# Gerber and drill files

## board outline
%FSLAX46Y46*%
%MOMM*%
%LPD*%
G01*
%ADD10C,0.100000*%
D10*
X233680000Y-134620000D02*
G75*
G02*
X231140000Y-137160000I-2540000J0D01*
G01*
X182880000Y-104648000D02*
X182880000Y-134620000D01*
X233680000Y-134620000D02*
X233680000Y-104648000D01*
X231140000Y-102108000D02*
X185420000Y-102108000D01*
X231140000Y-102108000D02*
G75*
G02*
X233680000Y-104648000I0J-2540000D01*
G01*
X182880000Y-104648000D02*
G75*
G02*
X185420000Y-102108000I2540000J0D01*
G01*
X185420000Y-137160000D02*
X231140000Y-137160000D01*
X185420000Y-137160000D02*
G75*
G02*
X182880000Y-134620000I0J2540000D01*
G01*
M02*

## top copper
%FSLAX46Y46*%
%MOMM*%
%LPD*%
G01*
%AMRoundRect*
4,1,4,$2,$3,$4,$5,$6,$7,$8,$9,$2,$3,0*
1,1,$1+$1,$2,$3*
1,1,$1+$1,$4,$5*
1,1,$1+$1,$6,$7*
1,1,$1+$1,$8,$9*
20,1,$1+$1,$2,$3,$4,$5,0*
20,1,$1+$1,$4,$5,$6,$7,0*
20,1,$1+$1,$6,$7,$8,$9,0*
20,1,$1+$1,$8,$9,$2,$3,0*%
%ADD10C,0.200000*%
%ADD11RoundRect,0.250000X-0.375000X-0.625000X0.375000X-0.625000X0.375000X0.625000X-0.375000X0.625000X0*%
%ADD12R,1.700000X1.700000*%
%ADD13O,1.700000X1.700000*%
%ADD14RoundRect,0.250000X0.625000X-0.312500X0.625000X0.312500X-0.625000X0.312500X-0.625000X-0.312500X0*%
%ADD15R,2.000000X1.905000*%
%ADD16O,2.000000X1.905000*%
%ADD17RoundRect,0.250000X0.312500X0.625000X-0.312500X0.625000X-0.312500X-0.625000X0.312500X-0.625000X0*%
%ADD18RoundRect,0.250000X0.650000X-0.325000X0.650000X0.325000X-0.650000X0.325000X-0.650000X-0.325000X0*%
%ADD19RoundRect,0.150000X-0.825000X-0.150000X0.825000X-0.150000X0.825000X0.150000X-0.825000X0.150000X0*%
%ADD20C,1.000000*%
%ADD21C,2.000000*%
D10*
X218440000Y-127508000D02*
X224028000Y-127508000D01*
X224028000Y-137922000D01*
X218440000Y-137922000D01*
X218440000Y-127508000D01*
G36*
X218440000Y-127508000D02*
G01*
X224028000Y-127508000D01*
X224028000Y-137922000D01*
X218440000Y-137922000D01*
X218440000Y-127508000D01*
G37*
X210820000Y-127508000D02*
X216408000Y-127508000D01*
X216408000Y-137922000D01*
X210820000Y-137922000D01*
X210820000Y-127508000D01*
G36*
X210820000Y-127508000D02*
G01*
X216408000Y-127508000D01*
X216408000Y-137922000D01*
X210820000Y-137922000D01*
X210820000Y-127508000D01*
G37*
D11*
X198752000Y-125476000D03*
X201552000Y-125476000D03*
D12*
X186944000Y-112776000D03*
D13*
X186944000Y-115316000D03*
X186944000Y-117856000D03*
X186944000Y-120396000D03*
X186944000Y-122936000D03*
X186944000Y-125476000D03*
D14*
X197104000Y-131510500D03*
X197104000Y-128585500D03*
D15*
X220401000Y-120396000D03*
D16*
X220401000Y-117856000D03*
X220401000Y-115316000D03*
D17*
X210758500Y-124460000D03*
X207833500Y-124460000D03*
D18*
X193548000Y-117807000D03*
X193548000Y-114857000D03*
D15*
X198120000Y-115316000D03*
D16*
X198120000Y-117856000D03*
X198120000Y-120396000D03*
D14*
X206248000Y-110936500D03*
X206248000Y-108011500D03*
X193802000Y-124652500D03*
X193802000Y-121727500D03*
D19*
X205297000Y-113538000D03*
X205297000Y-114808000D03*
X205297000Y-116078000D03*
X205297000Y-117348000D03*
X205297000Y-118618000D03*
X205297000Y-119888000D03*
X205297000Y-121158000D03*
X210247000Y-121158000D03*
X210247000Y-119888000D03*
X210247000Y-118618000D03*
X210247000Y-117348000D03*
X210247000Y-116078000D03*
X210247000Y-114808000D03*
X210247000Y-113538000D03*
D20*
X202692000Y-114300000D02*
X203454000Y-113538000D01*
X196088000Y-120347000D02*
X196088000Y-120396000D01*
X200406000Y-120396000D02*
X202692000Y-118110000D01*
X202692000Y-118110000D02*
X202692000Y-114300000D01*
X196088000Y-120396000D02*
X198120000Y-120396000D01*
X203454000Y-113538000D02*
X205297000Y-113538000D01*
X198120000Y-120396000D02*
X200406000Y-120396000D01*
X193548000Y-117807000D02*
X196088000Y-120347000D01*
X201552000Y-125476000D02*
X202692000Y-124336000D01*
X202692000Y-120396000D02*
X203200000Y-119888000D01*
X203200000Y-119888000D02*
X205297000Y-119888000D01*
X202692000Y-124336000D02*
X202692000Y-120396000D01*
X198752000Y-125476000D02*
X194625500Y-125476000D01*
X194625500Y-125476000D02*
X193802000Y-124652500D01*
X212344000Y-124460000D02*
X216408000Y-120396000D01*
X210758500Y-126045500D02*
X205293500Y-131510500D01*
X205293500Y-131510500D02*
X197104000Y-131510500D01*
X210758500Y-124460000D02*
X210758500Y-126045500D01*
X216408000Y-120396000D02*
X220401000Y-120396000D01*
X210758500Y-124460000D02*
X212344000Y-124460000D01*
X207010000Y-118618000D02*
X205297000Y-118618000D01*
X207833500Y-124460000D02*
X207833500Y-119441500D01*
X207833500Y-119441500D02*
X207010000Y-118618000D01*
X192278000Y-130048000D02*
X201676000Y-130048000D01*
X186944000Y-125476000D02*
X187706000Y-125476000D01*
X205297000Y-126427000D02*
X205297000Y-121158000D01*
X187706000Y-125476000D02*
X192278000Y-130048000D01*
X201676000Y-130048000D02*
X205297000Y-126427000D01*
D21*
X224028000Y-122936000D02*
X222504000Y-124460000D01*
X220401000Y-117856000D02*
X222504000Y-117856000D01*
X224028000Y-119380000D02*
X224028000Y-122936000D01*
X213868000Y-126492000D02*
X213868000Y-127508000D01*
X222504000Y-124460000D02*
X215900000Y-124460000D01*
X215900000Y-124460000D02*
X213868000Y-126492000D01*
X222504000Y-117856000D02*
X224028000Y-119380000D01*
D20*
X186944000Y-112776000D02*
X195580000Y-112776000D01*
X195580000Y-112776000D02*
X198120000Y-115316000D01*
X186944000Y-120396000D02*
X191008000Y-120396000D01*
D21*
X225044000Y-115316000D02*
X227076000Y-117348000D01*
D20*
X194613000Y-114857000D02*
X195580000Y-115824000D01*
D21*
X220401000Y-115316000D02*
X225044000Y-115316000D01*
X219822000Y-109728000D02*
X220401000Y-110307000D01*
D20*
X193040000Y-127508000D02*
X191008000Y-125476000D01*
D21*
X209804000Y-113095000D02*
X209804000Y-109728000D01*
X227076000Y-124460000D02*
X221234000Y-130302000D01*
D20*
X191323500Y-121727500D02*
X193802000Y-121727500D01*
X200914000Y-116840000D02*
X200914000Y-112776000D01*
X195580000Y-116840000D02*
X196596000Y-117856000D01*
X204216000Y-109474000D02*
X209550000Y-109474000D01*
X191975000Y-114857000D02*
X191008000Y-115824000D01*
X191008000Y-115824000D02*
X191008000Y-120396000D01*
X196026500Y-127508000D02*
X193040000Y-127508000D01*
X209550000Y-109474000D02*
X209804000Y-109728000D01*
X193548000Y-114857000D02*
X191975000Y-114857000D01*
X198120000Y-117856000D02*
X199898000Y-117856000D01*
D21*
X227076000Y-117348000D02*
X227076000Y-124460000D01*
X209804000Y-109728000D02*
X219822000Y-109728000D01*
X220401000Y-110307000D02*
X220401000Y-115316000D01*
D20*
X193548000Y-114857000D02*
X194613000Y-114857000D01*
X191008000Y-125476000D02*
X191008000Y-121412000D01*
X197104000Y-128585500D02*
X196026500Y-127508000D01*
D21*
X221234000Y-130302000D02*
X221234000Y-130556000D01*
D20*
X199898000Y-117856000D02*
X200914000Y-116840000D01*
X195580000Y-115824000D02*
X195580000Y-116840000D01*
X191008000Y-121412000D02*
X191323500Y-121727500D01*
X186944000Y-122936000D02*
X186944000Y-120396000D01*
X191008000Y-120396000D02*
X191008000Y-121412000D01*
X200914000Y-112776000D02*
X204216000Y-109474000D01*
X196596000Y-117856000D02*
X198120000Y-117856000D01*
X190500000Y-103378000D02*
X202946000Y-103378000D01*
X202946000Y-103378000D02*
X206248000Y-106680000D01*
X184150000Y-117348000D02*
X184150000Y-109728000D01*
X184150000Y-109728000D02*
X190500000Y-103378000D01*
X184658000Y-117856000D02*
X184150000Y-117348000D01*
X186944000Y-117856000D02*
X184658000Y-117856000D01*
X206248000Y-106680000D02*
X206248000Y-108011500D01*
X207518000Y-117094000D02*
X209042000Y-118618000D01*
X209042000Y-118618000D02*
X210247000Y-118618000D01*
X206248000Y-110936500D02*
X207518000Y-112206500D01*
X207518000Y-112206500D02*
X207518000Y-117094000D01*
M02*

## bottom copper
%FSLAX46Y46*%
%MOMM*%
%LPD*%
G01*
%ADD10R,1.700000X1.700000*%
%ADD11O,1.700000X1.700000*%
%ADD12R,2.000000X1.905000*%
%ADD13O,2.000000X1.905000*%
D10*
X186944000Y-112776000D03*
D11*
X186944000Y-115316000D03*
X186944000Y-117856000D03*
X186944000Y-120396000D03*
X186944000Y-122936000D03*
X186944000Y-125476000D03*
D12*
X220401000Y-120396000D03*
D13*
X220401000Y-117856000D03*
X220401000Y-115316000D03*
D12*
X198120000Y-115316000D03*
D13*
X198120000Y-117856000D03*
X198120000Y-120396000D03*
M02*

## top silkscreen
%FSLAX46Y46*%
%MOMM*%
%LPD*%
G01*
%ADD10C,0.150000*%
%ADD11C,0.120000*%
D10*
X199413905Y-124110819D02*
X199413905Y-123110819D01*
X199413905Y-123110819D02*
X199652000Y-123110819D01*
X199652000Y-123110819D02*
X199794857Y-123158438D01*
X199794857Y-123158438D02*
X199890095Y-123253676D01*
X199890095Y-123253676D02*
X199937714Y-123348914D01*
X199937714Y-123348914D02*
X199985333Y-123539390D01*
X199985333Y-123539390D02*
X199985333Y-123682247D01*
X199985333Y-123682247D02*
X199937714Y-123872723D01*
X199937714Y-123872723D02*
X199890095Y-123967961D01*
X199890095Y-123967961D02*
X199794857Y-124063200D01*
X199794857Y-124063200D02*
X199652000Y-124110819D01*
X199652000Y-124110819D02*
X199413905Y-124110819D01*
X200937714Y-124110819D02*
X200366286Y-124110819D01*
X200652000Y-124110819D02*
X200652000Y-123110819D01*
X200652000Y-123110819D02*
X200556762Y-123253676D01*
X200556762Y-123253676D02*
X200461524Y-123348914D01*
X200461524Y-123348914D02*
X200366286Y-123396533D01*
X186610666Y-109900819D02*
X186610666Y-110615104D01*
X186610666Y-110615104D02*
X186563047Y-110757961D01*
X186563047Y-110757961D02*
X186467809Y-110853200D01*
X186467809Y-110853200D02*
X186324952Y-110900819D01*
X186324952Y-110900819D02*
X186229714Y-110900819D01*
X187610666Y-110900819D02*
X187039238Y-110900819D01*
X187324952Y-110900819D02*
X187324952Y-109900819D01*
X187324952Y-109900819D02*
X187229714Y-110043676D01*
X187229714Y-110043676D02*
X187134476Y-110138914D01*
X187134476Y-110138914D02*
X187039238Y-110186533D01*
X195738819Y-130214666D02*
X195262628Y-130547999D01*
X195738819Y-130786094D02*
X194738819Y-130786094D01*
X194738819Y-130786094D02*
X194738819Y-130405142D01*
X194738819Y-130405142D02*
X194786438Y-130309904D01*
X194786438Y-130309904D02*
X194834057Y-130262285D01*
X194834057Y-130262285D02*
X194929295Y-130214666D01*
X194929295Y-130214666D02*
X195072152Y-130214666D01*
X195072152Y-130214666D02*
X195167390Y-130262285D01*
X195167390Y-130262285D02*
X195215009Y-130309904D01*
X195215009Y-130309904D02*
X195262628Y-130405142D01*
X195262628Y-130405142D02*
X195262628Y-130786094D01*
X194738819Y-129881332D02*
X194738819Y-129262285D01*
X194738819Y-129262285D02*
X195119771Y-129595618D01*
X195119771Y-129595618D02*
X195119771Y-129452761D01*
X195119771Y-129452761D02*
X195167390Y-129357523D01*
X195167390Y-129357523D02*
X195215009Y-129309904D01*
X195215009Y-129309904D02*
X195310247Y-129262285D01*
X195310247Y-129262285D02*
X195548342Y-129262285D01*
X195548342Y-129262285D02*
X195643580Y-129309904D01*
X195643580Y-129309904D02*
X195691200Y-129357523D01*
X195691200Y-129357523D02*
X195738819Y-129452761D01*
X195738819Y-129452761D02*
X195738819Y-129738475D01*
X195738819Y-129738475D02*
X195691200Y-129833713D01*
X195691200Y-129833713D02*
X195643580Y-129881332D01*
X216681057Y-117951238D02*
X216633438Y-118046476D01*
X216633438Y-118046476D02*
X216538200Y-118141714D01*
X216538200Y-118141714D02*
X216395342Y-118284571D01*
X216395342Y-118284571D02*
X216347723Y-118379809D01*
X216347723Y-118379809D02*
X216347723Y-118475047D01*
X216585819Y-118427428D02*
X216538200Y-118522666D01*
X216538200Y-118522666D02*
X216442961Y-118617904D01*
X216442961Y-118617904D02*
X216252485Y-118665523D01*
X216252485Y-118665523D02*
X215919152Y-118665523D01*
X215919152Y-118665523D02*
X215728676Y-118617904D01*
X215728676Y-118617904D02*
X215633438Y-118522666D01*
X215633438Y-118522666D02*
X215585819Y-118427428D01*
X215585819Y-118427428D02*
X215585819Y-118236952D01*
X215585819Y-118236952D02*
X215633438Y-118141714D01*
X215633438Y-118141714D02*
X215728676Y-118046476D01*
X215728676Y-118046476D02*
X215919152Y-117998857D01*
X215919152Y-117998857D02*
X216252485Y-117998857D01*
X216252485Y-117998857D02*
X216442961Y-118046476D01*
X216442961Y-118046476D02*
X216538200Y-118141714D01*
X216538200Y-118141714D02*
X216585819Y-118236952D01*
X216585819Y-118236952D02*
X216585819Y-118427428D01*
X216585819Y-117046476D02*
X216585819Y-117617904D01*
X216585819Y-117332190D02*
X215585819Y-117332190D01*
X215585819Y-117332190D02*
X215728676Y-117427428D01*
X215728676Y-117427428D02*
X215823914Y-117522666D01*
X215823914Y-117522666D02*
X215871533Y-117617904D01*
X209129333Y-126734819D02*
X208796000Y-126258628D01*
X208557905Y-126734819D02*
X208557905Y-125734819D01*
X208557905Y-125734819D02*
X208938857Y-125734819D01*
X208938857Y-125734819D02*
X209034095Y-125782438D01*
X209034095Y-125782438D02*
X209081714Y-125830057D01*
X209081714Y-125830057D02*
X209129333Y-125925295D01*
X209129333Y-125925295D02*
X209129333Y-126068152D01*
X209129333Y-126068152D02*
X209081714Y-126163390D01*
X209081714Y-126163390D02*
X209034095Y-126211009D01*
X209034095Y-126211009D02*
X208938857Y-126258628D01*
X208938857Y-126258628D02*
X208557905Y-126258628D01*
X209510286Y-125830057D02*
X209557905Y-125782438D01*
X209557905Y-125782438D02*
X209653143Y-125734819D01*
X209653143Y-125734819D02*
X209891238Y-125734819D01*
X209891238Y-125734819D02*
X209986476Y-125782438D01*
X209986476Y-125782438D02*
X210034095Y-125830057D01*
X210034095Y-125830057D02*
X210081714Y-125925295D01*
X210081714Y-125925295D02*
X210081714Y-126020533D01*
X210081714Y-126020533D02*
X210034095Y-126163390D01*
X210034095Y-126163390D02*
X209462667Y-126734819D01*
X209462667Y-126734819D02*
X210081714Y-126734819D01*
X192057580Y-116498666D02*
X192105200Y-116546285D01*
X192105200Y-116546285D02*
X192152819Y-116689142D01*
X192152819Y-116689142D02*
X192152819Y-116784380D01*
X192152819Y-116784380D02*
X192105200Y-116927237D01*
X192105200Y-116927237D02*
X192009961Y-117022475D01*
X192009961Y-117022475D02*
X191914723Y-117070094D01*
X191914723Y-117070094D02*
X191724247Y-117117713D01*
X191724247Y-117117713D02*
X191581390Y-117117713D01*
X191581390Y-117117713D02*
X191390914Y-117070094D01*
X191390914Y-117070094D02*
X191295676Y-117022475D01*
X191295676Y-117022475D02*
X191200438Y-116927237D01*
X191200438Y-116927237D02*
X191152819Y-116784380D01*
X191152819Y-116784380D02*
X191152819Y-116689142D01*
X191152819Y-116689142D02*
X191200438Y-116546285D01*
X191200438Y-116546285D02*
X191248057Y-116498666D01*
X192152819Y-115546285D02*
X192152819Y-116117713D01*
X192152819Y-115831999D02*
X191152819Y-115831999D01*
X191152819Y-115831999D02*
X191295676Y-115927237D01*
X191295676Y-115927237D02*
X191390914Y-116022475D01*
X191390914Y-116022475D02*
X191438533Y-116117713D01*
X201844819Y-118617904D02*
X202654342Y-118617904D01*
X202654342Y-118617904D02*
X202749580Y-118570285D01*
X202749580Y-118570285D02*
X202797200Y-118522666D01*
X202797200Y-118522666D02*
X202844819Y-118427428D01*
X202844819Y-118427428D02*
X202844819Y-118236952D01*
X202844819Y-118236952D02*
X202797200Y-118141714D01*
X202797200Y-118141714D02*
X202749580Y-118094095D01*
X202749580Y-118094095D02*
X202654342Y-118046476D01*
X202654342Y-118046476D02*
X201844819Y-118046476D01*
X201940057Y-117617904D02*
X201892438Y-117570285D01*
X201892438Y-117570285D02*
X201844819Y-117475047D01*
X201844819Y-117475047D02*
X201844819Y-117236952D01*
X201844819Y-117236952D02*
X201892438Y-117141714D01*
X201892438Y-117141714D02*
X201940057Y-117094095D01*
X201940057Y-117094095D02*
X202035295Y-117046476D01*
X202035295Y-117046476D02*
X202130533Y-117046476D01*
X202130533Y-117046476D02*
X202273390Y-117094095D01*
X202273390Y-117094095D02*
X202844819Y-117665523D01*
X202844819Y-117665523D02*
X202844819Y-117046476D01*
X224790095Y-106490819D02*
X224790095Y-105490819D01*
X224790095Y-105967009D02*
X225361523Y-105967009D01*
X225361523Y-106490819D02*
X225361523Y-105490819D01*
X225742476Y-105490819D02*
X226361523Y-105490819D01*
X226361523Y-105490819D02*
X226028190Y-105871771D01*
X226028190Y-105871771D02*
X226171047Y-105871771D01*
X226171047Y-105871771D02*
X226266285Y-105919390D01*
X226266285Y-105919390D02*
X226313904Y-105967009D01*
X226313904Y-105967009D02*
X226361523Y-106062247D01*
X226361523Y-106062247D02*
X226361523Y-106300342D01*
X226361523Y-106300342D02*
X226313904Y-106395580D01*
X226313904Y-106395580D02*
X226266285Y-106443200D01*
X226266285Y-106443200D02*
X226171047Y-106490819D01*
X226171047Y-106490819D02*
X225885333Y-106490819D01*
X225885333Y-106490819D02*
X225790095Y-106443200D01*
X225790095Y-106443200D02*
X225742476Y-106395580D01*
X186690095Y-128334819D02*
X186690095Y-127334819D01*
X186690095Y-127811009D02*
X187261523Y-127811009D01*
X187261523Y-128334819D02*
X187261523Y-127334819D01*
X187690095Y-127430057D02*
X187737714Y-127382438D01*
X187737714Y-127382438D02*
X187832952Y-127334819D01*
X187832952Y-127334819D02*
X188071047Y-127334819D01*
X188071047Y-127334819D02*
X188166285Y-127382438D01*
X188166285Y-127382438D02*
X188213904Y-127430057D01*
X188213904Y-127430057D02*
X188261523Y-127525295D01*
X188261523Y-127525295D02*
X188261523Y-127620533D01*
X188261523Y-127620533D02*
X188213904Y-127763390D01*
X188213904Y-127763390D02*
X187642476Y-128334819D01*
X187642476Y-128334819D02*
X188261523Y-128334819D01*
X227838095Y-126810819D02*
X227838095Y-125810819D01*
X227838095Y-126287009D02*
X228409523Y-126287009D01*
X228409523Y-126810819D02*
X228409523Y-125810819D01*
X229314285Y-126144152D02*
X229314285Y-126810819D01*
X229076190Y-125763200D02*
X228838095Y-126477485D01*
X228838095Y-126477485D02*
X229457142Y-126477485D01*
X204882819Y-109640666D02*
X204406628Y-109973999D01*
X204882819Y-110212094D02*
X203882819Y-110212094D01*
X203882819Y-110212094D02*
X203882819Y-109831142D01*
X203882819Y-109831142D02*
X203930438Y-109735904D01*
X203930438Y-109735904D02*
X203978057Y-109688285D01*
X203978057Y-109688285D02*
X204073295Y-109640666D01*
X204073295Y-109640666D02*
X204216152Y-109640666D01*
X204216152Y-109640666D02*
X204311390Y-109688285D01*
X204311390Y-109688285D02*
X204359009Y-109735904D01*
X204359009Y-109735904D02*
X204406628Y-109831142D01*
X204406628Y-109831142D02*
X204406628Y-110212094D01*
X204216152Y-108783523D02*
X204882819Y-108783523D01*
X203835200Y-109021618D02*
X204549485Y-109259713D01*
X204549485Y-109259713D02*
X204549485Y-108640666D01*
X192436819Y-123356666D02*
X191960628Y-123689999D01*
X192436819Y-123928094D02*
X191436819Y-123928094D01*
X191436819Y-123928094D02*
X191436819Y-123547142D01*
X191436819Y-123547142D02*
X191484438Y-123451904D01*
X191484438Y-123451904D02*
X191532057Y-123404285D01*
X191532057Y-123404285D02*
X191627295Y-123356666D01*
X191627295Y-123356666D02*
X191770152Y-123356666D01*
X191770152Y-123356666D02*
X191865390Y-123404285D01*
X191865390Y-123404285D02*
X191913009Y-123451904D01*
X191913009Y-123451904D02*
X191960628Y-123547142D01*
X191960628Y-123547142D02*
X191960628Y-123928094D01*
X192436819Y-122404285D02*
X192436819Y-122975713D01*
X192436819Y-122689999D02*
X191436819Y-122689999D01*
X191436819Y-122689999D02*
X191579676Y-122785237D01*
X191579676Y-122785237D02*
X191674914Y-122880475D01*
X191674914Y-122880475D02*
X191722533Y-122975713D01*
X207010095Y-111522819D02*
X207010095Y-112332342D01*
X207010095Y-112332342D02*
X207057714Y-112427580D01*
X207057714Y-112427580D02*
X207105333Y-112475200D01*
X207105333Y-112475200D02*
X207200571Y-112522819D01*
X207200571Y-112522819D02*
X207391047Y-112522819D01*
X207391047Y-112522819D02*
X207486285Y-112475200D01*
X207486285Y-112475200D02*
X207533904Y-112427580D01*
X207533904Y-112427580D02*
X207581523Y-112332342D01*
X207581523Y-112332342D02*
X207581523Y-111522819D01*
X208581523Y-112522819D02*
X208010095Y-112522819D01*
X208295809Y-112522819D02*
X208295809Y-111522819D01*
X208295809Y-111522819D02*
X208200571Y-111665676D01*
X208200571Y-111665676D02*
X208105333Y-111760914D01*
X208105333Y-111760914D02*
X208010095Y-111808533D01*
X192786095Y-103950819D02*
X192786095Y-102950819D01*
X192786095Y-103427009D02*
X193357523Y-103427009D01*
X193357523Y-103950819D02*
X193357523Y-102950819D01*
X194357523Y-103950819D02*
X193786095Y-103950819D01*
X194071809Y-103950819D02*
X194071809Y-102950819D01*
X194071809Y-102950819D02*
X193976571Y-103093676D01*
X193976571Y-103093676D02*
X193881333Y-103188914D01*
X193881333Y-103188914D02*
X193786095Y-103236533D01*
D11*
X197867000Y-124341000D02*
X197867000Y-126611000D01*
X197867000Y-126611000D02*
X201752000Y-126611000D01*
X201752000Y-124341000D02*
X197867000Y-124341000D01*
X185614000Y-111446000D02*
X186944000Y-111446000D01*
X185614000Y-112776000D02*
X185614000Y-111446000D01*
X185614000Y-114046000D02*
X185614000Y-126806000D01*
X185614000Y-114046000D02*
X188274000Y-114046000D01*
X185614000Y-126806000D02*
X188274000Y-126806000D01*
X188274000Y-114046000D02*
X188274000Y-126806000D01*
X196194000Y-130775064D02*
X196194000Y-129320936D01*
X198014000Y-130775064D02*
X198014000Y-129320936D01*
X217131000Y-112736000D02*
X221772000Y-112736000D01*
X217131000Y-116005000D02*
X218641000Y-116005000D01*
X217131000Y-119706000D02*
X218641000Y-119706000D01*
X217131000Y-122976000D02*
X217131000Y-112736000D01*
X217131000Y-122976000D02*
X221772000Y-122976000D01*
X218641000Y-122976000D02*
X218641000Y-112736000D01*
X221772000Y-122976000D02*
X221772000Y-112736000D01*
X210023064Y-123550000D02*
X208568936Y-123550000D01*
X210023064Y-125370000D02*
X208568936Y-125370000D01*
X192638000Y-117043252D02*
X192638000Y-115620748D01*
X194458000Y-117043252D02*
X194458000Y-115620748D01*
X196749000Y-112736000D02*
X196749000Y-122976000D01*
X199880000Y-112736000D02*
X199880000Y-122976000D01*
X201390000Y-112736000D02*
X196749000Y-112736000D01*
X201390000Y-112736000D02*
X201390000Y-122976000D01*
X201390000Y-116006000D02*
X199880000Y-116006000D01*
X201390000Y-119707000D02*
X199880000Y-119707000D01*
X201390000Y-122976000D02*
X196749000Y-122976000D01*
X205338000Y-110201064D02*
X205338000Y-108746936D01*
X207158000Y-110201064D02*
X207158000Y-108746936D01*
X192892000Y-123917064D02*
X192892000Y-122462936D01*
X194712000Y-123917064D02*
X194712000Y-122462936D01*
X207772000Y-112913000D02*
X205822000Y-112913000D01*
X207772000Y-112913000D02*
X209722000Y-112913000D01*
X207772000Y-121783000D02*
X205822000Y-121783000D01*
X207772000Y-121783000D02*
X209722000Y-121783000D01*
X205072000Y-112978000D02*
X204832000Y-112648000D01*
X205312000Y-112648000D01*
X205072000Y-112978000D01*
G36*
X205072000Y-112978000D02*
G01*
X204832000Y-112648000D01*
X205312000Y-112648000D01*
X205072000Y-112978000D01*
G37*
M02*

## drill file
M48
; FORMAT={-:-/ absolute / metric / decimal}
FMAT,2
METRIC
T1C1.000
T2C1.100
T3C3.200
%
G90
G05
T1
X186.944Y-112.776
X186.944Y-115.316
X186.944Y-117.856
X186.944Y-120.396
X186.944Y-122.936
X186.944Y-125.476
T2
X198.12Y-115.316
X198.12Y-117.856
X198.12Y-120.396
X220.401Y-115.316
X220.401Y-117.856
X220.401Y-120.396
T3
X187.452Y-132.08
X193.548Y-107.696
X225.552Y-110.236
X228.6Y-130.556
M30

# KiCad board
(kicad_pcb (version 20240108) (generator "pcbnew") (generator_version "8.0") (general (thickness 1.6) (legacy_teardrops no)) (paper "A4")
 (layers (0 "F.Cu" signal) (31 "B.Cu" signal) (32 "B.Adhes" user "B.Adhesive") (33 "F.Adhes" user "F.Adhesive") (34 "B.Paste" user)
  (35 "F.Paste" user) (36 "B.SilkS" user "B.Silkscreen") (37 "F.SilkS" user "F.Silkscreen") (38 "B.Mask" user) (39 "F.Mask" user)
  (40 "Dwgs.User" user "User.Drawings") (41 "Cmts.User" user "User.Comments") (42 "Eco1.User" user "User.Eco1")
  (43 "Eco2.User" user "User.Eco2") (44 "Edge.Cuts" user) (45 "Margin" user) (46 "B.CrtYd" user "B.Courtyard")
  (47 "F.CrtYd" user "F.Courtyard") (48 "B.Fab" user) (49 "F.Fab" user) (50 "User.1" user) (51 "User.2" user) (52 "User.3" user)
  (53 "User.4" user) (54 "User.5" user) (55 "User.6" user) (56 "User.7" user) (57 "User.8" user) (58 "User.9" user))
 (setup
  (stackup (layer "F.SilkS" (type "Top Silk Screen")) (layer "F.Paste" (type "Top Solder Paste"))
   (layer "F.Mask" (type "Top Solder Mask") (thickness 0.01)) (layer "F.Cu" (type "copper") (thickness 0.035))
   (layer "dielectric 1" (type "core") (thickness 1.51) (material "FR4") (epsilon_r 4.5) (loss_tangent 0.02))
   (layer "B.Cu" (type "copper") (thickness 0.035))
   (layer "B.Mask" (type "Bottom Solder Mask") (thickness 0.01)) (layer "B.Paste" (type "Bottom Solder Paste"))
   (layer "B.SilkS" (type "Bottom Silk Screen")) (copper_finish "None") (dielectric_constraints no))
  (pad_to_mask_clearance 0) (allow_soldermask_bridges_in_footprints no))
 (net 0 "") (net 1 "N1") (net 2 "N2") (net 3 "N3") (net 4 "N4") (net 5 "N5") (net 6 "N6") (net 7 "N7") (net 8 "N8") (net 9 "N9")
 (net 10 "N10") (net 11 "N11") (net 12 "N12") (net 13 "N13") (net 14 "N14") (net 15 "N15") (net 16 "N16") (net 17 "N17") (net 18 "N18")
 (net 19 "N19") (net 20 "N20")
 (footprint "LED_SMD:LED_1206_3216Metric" (layer "F.Cu") (at 200.152 125.476)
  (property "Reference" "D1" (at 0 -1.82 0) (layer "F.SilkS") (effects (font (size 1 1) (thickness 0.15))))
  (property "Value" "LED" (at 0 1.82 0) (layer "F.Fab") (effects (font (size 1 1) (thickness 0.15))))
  (fp_line (start -2.285 -1.135) (end -2.285 1.135) (stroke (width 0.12) (type solid)) (layer "F.SilkS"))
  (fp_line (start -2.285 1.135) (end 1.6 1.135) (stroke (width 0.12) (type solid)) (layer "F.SilkS"))
  (fp_line (start 1.6 -1.135) (end -2.285 -1.135) (stroke (width 0.12) (type solid)) (layer "F.SilkS"))
  (pad "1" smd roundrect (at -1.4 0) (size 1.25 1.75) (layers "F.Cu" "F.Paste" "F.Mask") (roundrect_rratio 0.2) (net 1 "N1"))
  (pad "2" smd roundrect (at 1.4 0) (size 1.25 1.75) (layers "F.Cu" "F.Paste" "F.Mask") (roundrect_rratio 0.2) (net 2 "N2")))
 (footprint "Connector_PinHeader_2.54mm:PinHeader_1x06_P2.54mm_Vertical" (layer "F.Cu") (at 186.944 112.776)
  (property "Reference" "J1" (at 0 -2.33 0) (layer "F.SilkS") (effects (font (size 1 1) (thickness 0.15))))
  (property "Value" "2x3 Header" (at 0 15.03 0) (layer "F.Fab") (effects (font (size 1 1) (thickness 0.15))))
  (fp_line (start -1.33 -1.33) (end 0 -1.33) (stroke (width 0.12) (type solid)) (layer "F.SilkS"))
  (fp_line (start -1.33 0) (end -1.33 -1.33) (stroke (width 0.12) (type solid)) (layer "F.SilkS"))
  (fp_line (start -1.33 1.27) (end -1.33 14.03) (stroke (width 0.12) (type solid)) (layer "F.SilkS"))
  (fp_line (start -1.33 1.27) (end 1.33 1.27) (stroke (width 0.12) (type solid)) (layer "F.SilkS"))
  (fp_line (start -1.33 14.03) (end 1.33 14.03) (stroke (width 0.12) (type solid)) (layer "F.SilkS"))
  (fp_line (start 1.33 1.27) (end 1.33 14.03) (stroke (width 0.12) (type solid)) (layer "F.SilkS"))
  (pad "1" thru_hole rect (at 0 0) (size 1.7 1.7) (drill 1) (layers "*.Cu" "*.Mask") (remove_unused_layers no) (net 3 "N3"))
  (pad "2" thru_hole oval (at 0 2.54) (size 1.7 1.7) (drill 1) (layers "*.Cu" "*.Mask") (remove_unused_layers no) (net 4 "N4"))
  (pad "3" thru_hole oval (at 0 5.08) (size 1.7 1.7) (drill 1) (layers "*.Cu" "*.Mask") (remove_unused_layers no) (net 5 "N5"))
  (pad "4" thru_hole oval (at 0 7.62) (size 1.7 1.7) (drill 1) (layers "*.Cu" "*.Mask") (remove_unused_layers no) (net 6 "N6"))
  (pad "5" thru_hole oval (at 0 10.16) (size 1.7 1.7) (drill 1) (layers "*.Cu" "*.Mask") (remove_unused_layers no) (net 6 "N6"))
  (pad "6" thru_hole oval (at 0 12.7) (size 1.7 1.7) (drill 1) (layers "*.Cu" "*.Mask") (remove_unused_layers no) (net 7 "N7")))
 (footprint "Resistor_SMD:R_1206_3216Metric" (layer "F.Cu") (at 197.104 130.048 90)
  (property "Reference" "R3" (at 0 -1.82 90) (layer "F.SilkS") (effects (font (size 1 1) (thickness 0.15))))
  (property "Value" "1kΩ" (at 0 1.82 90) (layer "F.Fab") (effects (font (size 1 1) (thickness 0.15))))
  (fp_line (start -0.727064 -0.91) (end 0.727064 -0.91) (stroke (width 0.12) (type solid)) (layer "F.SilkS"))
  (fp_line (start -0.727064 0.91) (end 0.727064 0.91) (stroke (width 0.12) (type solid)) (layer "F.SilkS"))
  (pad "1" smd roundrect (at -1.4625 0 90) (size 1.125 1.75) (layers "F.Cu" "F.Paste" "F.Mask") (roundrect_rratio 0.222222) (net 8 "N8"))
  (pad "2" smd roundrect (at 1.4625 0 90) (size 1.125 1.75) (layers "F.Cu" "F.Paste" "F.Mask") (roundrect_rratio 0.222222) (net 6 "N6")))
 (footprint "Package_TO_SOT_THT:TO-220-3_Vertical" (layer "F.Cu") (at 220.401 120.396 90)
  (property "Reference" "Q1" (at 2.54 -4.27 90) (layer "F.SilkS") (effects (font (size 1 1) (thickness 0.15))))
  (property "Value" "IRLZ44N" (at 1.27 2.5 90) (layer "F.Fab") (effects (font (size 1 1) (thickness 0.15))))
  (fp_line (start 7.66 -3.27) (end 7.66 1.371) (stroke (width 0.12) (type solid)) (layer "F.SilkS"))
  (fp_line (start 4.391 -3.27) (end 4.391 -1.76) (stroke (width 0.12) (type solid)) (layer "F.SilkS"))
  (fp_line (start 0.69 -3.27) (end 0.69 -1.76) (stroke (width 0.12) (type solid)) (layer "F.SilkS"))
  (fp_line (start -2.58 -3.27) (end 7.66 -3.27) (stroke (width 0.12) (type solid)) (layer "F.SilkS"))
  (fp_line (start -2.58 -3.27) (end -2.58 1.371) (stroke (width 0.12) (type solid)) (layer "F.SilkS"))
  (fp_line (start -2.58 -1.76) (end 7.66 -1.76) (stroke (width 0.12) (type solid)) (layer "F.SilkS"))
  (fp_line (start -2.58 1.371) (end 7.66 1.371) (stroke (width 0.12) (type solid)) (layer "F.SilkS"))
  (pad "1" thru_hole rect (at 0 0 90) (size 1.905 2) (drill 1.1) (layers "*.Cu" "*.Mask") (remove_unused_layers no) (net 8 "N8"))
  (pad "2" thru_hole oval (at 2.54 0 90) (size 1.905 2) (drill 1.1) (layers "*.Cu" "*.Mask") (remove_unused_layers no) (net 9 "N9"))
  (pad "3" thru_hole oval (at 5.08 0 90) (size 1.905 2) (drill 1.1) (layers "*.Cu" "*.Mask") (remove_unused_layers no) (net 6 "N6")))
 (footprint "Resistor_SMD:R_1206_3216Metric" (layer "F.Cu") (at 209.296 124.46 180)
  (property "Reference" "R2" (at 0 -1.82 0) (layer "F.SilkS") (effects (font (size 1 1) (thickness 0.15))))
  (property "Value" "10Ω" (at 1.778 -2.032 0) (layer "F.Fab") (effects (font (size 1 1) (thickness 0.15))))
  (fp_line (start -0.727064 0.91) (end 0.727064 0.91) (stroke (width 0.12) (type solid)) (layer "F.SilkS"))
  (fp_line (start -0.727064 -0.91) (end 0.727064 -0.91) (stroke (width 0.12) (type solid)) (layer "F.SilkS"))
  (pad "1" smd roundrect (at -1.4625 0 180) (size 1.125 1.75) (layers "F.Cu" "F.Paste" "F.Mask") (roundrect_rratio 0.222222) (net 8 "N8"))
  (pad "2" smd roundrect (at 1.4625 0 180) (size 1.125 1.75) (layers "F.Cu" "F.Paste" "F.Mask") (roundrect_rratio 0.222222) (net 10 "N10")))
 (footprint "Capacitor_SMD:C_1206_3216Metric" (layer "F.Cu") (at 193.548 116.332 90)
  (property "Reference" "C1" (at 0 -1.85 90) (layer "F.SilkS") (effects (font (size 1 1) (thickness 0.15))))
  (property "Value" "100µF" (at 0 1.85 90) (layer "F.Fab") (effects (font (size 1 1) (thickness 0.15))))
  (fp_line (start -0.711252 -0.91) (end 0.711252 -0.91) (stroke (width 0.12) (type solid)) (layer "F.SilkS"))
  (fp_line (start -0.711252 0.91) (end 0.711252 0.91) (stroke (width 0.12) (type solid)) (layer "F.SilkS"))
  (pad "1" smd roundrect (at -1.475 0 90) (size 1.15 1.8) (layers "F.Cu" "F.Paste" "F.Mask") (roundrect_rratio 0.217391) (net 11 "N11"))
  (pad "2" smd roundrect (at 1.475 0 90) (size 1.15 1.8) (layers "F.Cu" "F.Paste" "F.Mask") (roundrect_rratio 0.217391) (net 6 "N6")))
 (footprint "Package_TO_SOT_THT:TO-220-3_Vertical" (layer "F.Cu") (at 198.12 115.316 -90)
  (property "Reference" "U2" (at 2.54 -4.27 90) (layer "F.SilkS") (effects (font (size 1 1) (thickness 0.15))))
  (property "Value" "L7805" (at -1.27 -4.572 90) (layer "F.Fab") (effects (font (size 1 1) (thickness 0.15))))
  (fp_line (start -2.58 1.371) (end 7.66 1.371) (stroke (width 0.12) (type solid)) (layer "F.SilkS"))
  (fp_line (start -2.58 -1.76) (end 7.66 -1.76) (stroke (width 0.12) (type solid)) (layer "F.SilkS"))
  (fp_line (start -2.58 -3.27) (end -2.58 1.371) (stroke (width 0.12) (type solid)) (layer "F.SilkS"))
  (fp_line (start -2.58 -3.27) (end 7.66 -3.27) (stroke (width 0.12) (type solid)) (layer "F.SilkS"))
  (fp_line (start 0.69 -3.27) (end 0.69 -1.76) (stroke (width 0.12) (type solid)) (layer "F.SilkS"))
  (fp_line (start 4.391 -3.27) (end 4.391 -1.76) (stroke (width 0.12) (type solid)) (layer "F.SilkS"))
  (fp_line (start 7.66 -3.27) (end 7.66 1.371) (stroke (width 0.12) (type solid)) (layer "F.SilkS"))
  (pad "1" thru_hole rect (at 0 0 270) (size 1.905 2) (drill 1.1) (layers "*.Cu" "*.Mask") (remove_unused_layers no) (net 3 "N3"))
  (pad "2" thru_hole oval (at 2.54 0 270) (size 1.905 2) (drill 1.1) (layers "*.Cu" "*.Mask") (remove_unused_layers no) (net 6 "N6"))
  (pad "3" thru_hole oval (at 5.08 0 270) (size 1.905 2) (drill 1.1) (layers "*.Cu" "*.Mask") (remove_unused_layers no) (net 11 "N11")))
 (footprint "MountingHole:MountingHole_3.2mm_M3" (layer "F.Cu") (at 225.552 110.236)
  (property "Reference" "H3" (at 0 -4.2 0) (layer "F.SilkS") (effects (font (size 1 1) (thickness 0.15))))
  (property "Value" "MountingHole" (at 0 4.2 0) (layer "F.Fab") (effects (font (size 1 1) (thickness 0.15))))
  (pad "" np_thru_hole circle (at 0 0) (size 3.2 3.2) (drill 3.2) (layers "*.Cu" "*.Mask")))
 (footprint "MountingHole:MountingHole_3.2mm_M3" (layer "F.Cu") (at 187.452 132.08)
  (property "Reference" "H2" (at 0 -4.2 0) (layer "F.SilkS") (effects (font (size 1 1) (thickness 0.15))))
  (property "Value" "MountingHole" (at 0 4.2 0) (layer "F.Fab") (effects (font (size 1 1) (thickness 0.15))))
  (pad "" np_thru_hole circle (at 0 0) (size 3.2 3.2) (drill 3.2) (layers "*.Cu" "*.Mask")))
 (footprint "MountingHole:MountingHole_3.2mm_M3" (layer "F.Cu") (at 228.6 130.556)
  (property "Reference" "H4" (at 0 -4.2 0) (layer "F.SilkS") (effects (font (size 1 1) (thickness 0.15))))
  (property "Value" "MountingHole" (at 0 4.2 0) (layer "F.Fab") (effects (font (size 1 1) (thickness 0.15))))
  (pad "" np_thru_hole circle (at 0 0) (size 3.2 3.2) (drill 3.2) (layers "*.Cu" "*.Mask")))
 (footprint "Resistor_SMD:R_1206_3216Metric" (layer "F.Cu") (at 206.248 109.474 90)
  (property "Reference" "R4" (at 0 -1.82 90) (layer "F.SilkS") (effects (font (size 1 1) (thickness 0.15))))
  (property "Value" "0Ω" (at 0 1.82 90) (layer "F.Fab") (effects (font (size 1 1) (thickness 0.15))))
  (fp_line (start -0.727064 -0.91) (end 0.727064 -0.91) (stroke (width 0.12) (type solid)) (layer "F.SilkS"))
  (fp_line (start -0.727064 0.91) (end 0.727064 0.91) (stroke (width 0.12) (type solid)) (layer "F.SilkS"))
  (pad "1" smd roundrect (at -1.4625 0 90) (size 1.125 1.75) (layers "F.Cu" "F.Paste" "F.Mask") (roundrect_rratio 0.222222) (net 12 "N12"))
  (pad "2" smd roundrect (at 1.4625 0 90) (size 1.125 1.75) (layers "F.Cu" "F.Paste" "F.Mask") (roundrect_rratio 0.222222) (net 5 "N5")))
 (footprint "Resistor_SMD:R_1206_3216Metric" (layer "F.Cu") (at 193.802 123.19 90)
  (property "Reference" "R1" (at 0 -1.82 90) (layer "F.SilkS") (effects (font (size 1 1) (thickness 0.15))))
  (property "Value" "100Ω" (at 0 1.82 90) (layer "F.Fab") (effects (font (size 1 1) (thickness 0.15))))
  (fp_line (start -0.727064 -0.91) (end 0.727064 -0.91) (stroke (width 0.12) (type solid)) (layer "F.SilkS"))
  (fp_line (start -0.727064 0.91) (end 0.727064 0.91) (stroke (width 0.12) (type solid)) (layer "F.SilkS"))
  (pad "1" smd roundrect (at -1.4625 0 90) (size 1.125 1.75) (layers "F.Cu" "F.Paste" "F.Mask") (roundrect_rratio 0.222222) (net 1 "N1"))
  (pad "2" smd roundrect (at 1.4625 0 90) (size 1.125 1.75) (layers "F.Cu" "F.Paste" "F.Mask") (roundrect_rratio 0.222222) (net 6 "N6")))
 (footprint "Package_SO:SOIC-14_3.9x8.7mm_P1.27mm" (layer "F.Cu") (at 207.772 117.348)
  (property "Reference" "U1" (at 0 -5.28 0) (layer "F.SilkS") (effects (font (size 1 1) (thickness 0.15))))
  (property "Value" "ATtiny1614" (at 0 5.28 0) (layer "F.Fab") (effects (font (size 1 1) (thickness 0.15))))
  (fp_line (start 0 -4.435) (end -1.95 -4.435) (stroke (width 0.12) (type solid)) (layer "F.SilkS"))
  (fp_line (start 0 -4.435) (end 1.95 -4.435) (stroke (width 0.12) (type solid)) (layer "F.SilkS"))
  (fp_line (start 0 4.435) (end -1.95 4.435) (stroke (width 0.12) (type solid)) (layer "F.SilkS"))
  (fp_line (start 0 4.435) (end 1.95 4.435) (stroke (width 0.12) (type solid)) (layer "F.SilkS"))
  (fp_poly
   (pts (xy -2.7 -4.37) (xy -2.94 -4.7) (xy -2.46 -4.7) (xy -2.7 -4.37)) (stroke (width 0.12) (type solid)) (fill solid) (layer "F.SilkS"))
  (pad "1" smd roundrect (at -2.475 -3.81) (size 1.95 0.6) (layers "F.Cu" "F.Paste" "F.Mask") (roundrect_rratio 0.25) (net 11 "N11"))
  (pad "2" smd roundrect (at -2.475 -2.54) (size 1.95 0.6) (layers "F.Cu" "F.Paste" "F.Mask") (roundrect_rratio 0.25) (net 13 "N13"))
  (pad "3" smd roundrect (at -2.475 -1.27) (size 1.95 0.6) (layers "F.Cu" "F.Paste" "F.Mask") (roundrect_rratio 0.25) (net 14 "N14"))
  (pad "4" smd roundrect (at -2.475 0) (size 1.95 0.6) (layers "F.Cu" "F.Paste" "F.Mask") (roundrect_rratio 0.25) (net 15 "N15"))
  (pad "5" smd roundrect (at -2.475 1.27) (size 1.95 0.6) (layers "F.Cu" "F.Paste" "F.Mask") (roundrect_rratio 0.25) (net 10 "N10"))
  (pad "6" smd roundrect (at -2.475 2.54) (size 1.95 0.6) (layers "F.Cu" "F.Paste" "F.Mask") (roundrect_rratio 0.25) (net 2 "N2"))
  (pad "7" smd roundrect (at -2.475 3.81) (size 1.95 0.6) (layers "F.Cu" "F.Paste" "F.Mask") (roundrect_rratio 0.25) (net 7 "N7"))
  (pad "8" smd roundrect (at 2.475 3.81) (size 1.95 0.6) (layers "F.Cu" "F.Paste" "F.Mask") (roundrect_rratio 0.25) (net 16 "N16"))
  (pad "9" smd roundrect (at 2.475 2.54) (size 1.95 0.6) (layers "F.Cu" "F.Paste" "F.Mask") (roundrect_rratio 0.25) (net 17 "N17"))
  (pad "10" smd roundrect (at 2.475 1.27) (size 1.95 0.6) (layers "F.Cu" "F.Paste" "F.Mask") (roundrect_rratio 0.25) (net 12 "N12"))
  (pad "11" smd roundrect (at 2.475 0) (size 1.95 0.6) (layers "F.Cu" "F.Paste" "F.Mask") (roundrect_rratio 0.25) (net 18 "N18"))
  (pad "12" smd roundrect (at 2.475 -1.27) (size 1.95 0.6) (layers "F.Cu" "F.Paste" "F.Mask") (roundrect_rratio 0.25) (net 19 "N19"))
  (pad "13" smd roundrect (at 2.475 -2.54) (size 1.95 0.6) (layers "F.Cu" "F.Paste" "F.Mask") (roundrect_rratio 0.25) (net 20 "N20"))
  (pad "14" smd roundrect (at 2.475 -3.81) (size 1.95 0.6) (layers "F.Cu" "F.Paste" "F.Mask") (roundrect_rratio 0.25) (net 6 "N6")))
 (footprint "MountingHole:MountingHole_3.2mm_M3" (layer "F.Cu") (at 193.548 107.696)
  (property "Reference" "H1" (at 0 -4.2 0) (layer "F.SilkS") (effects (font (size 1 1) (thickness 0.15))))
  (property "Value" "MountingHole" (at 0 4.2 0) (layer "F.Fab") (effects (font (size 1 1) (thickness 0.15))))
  (pad "" np_thru_hole circle (at 0 0) (size 3.2 3.2) (drill 3.2) (layers "*.Cu" "*.Mask")))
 (gr_rect (start 218.44 127.508) (end 224.028 137.922) (stroke (width 0.2) (type solid)) (fill solid) (layer "F.Cu") (net 6))
 (gr_rect (start 210.82 127.508) (end 216.408 137.922) (stroke (width 0.2) (type solid)) (fill solid) (layer "F.Cu") (net 9))
 (gr_arc (start 233.68 134.62) (mid 232.936051 136.416051) (end 231.14 137.16) (stroke (width 0.1) (type default)) (layer "Edge.Cuts"))
 (gr_line (start 182.88 104.648) (end 182.88 134.62) (stroke (width 0.1) (type default)) (layer "Edge.Cuts"))
 (gr_line (start 233.68 134.62) (end 233.68 104.648) (stroke (width 0.1) (type default)) (layer "Edge.Cuts"))
 (gr_line (start 231.14 102.108) (end 185.42 102.108) (stroke (width 0.1) (type default)) (layer "Edge.Cuts"))
 (gr_arc (start 231.14 102.108) (mid 232.936051 102.851949) (end 233.68 104.648) (stroke (width 0.1) (type default)) (layer "Edge.Cuts"))
 (gr_arc (start 182.88 104.648) (mid 183.623949 102.851949) (end 185.42 102.108) (stroke (width 0.1) (type default)) (layer "Edge.Cuts"))
 (gr_line (start 185.42 137.16) (end 231.14 137.16) (stroke (width 0.1) (type default)) (layer "Edge.Cuts"))
 (gr_arc (start 185.42 137.16) (mid 183.623949 136.416051) (end 182.88 134.62) (stroke (width 0.1) (type default)) (layer "Edge.Cuts"))
 (segment (start 202.692 114.3) (end 203.454 113.538) (width 1) (layer "F.Cu") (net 11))
 (segment (start 196.088 120.347) (end 196.088 120.396) (width 1) (layer "F.Cu") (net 11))
 (segment (start 200.406 120.396) (end 202.692 118.11) (width 1) (layer "F.Cu") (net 11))
 (segment (start 202.692 118.11) (end 202.692 114.3) (width 1) (layer "F.Cu") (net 11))
 (segment (start 196.088 120.396) (end 198.12 120.396) (width 1) (layer "F.Cu") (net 11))
 (segment (start 203.454 113.538) (end 205.297 113.538) (width 1) (layer "F.Cu") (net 11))
 (segment (start 198.12 120.396) (end 200.406 120.396) (width 1) (layer "F.Cu") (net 11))
 (segment (start 193.548 117.807) (end 196.088 120.347) (width 1) (layer "F.Cu") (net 11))
 (segment (start 201.552 125.476) (end 202.692 124.336) (width 1) (layer "F.Cu") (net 2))
 (segment (start 202.692 120.396) (end 203.2 119.888) (width 1) (layer "F.Cu") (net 2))
 (segment (start 203.2 119.888) (end 205.297 119.888) (width 1) (layer "F.Cu") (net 2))
 (segment (start 202.692 124.336) (end 202.692 120.396) (width 1) (layer "F.Cu") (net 2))
 (segment (start 198.752 125.476) (end 194.6255 125.476) (width 1) (layer "F.Cu") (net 1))
 (segment (start 194.6255 125.476) (end 193.802 124.6525) (width 1) (layer "F.Cu") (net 1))
 (segment (start 212.344 124.46) (end 216.408 120.396) (width 1) (layer "F.Cu") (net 8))
 (segment (start 210.7585 126.0455) (end 205.2935 131.5105) (width 1) (layer "F.Cu") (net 8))
 (segment (start 205.2935 131.5105) (end 197.104 131.5105) (width 1) (layer "F.Cu") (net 8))
 (segment (start 210.7585 124.46) (end 210.7585 126.0455) (width 1) (layer "F.Cu") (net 8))
 (segment (start 216.408 120.396) (end 220.401 120.396) (width 1) (layer "F.Cu") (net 8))
 (segment (start 210.7585 124.46) (end 212.344 124.46) (width 1) (layer "F.Cu") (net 8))
 (segment (start 207.01 118.618) (end 205.297 118.618) (width 1) (layer "F.Cu") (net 10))
 (segment (start 207.8335 124.46) (end 207.8335 119.4415) (width 1) (layer "F.Cu") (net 10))
 (segment (start 207.8335 119.4415) (end 207.01 118.618) (width 1) (layer "F.Cu") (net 10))
 (segment (start 192.278 130.048) (end 201.676 130.048) (width 1) (layer "F.Cu") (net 7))
 (segment (start 186.944 125.476) (end 187.706 125.476) (width 1) (layer "F.Cu") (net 7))
 (segment (start 205.297 126.427) (end 205.297 121.158) (width 1) (layer "F.Cu") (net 7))
 (segment (start 187.706 125.476) (end 192.278 130.048) (width 1) (layer "F.Cu") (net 7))
 (segment (start 201.676 130.048) (end 205.297 126.427) (width 1) (layer "F.Cu") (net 7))
 (segment (start 224.028 122.936) (end 222.504 124.46) (width 2) (layer "F.Cu") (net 9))
 (segment (start 220.401 117.856) (end 222.504 117.856) (width 2) (layer "F.Cu") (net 9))
 (segment (start 224.028 119.38) (end 224.028 122.936) (width 2) (layer "F.Cu") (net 9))
 (segment (start 213.868 126.492) (end 213.868 127.508) (width 2) (layer "F.Cu") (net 9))
 (segment (start 222.504 124.46) (end 215.9 124.46) (width 2) (layer "F.Cu") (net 9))
 (segment (start 215.9 124.46) (end 213.868 126.492) (width 2) (layer "F.Cu") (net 9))
 (segment (start 222.504 117.856) (end 224.028 119.38) (width 2) (layer "F.Cu") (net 9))
 (segment (start 186.944 112.776) (end 195.58 112.776) (width 1) (layer "F.Cu") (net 3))
 (segment (start 195.58 112.776) (end 198.12 115.316) (width 1) (layer "F.Cu") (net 3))
 (segment (start 186.944 120.396) (end 191.008 120.396) (width 1) (layer "F.Cu") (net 6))
 (segment (start 225.044 115.316) (end 227.076 117.348) (width 2) (layer "F.Cu") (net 6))
 (segment (start 194.613 114.857) (end 195.58 115.824) (width 1) (layer "F.Cu") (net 6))
 (segment (start 220.401 115.316) (end 225.044 115.316) (width 2) (layer "F.Cu") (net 6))
 (segment (start 219.822 109.728) (end 220.401 110.307) (width 2) (layer "F.Cu") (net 6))
 (segment (start 193.04 127.508) (end 191.008 125.476) (width 1) (layer "F.Cu") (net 6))
 (segment (start 209.804 113.095) (end 209.804 109.728) (width 2) (layer "F.Cu") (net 6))
 (segment (start 227.076 124.46) (end 221.234 130.302) (width 2) (layer "F.Cu") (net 6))
 (segment (start 191.3235 121.7275) (end 193.802 121.7275) (width 1) (layer "F.Cu") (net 6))
 (segment (start 200.914 116.84) (end 200.914 112.776) (width 1) (layer "F.Cu") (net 6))
 (segment (start 195.58 116.84) (end 196.596 117.856) (width 1) (layer "F.Cu") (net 6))
 (segment (start 204.216 109.474) (end 209.55 109.474) (width 1) (layer "F.Cu") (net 6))
 (segment (start 191.975 114.857) (end 191.008 115.824) (width 1) (layer "F.Cu") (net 6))
 (segment (start 191.008 115.824) (end 191.008 120.396) (width 1) (layer "F.Cu") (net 6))
 (segment (start 196.0265 127.508) (end 193.04 127.508) (width 1) (layer "F.Cu") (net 6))
 (segment (start 209.55 109.474) (end 209.804 109.728) (width 1) (layer "F.Cu") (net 6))
 (segment (start 193.548 114.857) (end 191.975 114.857) (width 1) (layer "F.Cu") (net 6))
 (segment (start 198.12 117.856) (end 199.898 117.856) (width 1) (layer "F.Cu") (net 6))
 (segment (start 227.076 117.348) (end 227.076 124.46) (width 2) (layer "F.Cu") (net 6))
 (segment (start 209.804 109.728) (end 219.822 109.728) (width 2) (layer "F.Cu") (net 6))
 (segment (start 220.401 110.307) (end 220.401 115.316) (width 2) (layer "F.Cu") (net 6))
 (segment (start 193.548 114.857) (end 194.613 114.857) (width 1) (layer "F.Cu") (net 6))
 (segment (start 191.008 125.476) (end 191.008 121.412) (width 1) (layer "F.Cu") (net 6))
 (segment (start 197.104 128.5855) (end 196.0265 127.508) (width 1) (layer "F.Cu") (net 6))
 (segment (start 221.234 130.302) (end 221.234 130.556) (width 2) (layer "F.Cu") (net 6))
 (segment (start 199.898 117.856) (end 200.914 116.84) (width 1) (layer "F.Cu") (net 6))
 (segment (start 195.58 115.824) (end 195.58 116.84) (width 1) (layer "F.Cu") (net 6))
 (segment (start 191.008 121.412) (end 191.3235 121.7275) (width 1) (layer "F.Cu") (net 6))
 (segment (start 186.944 122.936) (end 186.944 120.396) (width 1) (layer "F.Cu") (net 6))
 (segment (start 191.008 120.396) (end 191.008 121.412) (width 1) (layer "F.Cu") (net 6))
 (segment (start 200.914 112.776) (end 204.216 109.474) (width 1) (layer "F.Cu") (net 6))
 (segment (start 196.596 117.856) (end 198.12 117.856) (width 1) (layer "F.Cu") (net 6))
 (segment (start 190.5 103.378) (end 202.946 103.378) (width 1) (layer "F.Cu") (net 5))
 (segment (start 202.946 103.378) (end 206.248 106.68) (width 1) (layer "F.Cu") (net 5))
 (segment (start 184.15 117.348) (end 184.15 109.728) (width 1) (layer "F.Cu") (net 5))
 (segment (start 184.15 109.728) (end 190.5 103.378) (width 1) (layer "F.Cu") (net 5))
 (segment (start 184.658 117.856) (end 184.15 117.348) (width 1) (layer "F.Cu") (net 5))
 (segment (start 186.944 117.856) (end 184.658 117.856) (width 1) (layer "F.Cu") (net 5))
 (segment (start 206.248 106.68) (end 206.248 108.0115) (width 1) (layer "F.Cu") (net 5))
 (segment (start 207.518 117.094) (end 209.042 118.618) (width 1) (layer "F.Cu") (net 12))
 (segment (start 209.042 118.618) (end 210.247 118.618) (width 1) (layer "F.Cu") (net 12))
 (segment (start 206.248 110.9365) (end 207.518 112.2065) (width 1) (layer "F.Cu") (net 12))
 (segment (start 207.518 112.2065) (end 207.518 117.094) (width 1) (layer "F.Cu") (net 12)))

